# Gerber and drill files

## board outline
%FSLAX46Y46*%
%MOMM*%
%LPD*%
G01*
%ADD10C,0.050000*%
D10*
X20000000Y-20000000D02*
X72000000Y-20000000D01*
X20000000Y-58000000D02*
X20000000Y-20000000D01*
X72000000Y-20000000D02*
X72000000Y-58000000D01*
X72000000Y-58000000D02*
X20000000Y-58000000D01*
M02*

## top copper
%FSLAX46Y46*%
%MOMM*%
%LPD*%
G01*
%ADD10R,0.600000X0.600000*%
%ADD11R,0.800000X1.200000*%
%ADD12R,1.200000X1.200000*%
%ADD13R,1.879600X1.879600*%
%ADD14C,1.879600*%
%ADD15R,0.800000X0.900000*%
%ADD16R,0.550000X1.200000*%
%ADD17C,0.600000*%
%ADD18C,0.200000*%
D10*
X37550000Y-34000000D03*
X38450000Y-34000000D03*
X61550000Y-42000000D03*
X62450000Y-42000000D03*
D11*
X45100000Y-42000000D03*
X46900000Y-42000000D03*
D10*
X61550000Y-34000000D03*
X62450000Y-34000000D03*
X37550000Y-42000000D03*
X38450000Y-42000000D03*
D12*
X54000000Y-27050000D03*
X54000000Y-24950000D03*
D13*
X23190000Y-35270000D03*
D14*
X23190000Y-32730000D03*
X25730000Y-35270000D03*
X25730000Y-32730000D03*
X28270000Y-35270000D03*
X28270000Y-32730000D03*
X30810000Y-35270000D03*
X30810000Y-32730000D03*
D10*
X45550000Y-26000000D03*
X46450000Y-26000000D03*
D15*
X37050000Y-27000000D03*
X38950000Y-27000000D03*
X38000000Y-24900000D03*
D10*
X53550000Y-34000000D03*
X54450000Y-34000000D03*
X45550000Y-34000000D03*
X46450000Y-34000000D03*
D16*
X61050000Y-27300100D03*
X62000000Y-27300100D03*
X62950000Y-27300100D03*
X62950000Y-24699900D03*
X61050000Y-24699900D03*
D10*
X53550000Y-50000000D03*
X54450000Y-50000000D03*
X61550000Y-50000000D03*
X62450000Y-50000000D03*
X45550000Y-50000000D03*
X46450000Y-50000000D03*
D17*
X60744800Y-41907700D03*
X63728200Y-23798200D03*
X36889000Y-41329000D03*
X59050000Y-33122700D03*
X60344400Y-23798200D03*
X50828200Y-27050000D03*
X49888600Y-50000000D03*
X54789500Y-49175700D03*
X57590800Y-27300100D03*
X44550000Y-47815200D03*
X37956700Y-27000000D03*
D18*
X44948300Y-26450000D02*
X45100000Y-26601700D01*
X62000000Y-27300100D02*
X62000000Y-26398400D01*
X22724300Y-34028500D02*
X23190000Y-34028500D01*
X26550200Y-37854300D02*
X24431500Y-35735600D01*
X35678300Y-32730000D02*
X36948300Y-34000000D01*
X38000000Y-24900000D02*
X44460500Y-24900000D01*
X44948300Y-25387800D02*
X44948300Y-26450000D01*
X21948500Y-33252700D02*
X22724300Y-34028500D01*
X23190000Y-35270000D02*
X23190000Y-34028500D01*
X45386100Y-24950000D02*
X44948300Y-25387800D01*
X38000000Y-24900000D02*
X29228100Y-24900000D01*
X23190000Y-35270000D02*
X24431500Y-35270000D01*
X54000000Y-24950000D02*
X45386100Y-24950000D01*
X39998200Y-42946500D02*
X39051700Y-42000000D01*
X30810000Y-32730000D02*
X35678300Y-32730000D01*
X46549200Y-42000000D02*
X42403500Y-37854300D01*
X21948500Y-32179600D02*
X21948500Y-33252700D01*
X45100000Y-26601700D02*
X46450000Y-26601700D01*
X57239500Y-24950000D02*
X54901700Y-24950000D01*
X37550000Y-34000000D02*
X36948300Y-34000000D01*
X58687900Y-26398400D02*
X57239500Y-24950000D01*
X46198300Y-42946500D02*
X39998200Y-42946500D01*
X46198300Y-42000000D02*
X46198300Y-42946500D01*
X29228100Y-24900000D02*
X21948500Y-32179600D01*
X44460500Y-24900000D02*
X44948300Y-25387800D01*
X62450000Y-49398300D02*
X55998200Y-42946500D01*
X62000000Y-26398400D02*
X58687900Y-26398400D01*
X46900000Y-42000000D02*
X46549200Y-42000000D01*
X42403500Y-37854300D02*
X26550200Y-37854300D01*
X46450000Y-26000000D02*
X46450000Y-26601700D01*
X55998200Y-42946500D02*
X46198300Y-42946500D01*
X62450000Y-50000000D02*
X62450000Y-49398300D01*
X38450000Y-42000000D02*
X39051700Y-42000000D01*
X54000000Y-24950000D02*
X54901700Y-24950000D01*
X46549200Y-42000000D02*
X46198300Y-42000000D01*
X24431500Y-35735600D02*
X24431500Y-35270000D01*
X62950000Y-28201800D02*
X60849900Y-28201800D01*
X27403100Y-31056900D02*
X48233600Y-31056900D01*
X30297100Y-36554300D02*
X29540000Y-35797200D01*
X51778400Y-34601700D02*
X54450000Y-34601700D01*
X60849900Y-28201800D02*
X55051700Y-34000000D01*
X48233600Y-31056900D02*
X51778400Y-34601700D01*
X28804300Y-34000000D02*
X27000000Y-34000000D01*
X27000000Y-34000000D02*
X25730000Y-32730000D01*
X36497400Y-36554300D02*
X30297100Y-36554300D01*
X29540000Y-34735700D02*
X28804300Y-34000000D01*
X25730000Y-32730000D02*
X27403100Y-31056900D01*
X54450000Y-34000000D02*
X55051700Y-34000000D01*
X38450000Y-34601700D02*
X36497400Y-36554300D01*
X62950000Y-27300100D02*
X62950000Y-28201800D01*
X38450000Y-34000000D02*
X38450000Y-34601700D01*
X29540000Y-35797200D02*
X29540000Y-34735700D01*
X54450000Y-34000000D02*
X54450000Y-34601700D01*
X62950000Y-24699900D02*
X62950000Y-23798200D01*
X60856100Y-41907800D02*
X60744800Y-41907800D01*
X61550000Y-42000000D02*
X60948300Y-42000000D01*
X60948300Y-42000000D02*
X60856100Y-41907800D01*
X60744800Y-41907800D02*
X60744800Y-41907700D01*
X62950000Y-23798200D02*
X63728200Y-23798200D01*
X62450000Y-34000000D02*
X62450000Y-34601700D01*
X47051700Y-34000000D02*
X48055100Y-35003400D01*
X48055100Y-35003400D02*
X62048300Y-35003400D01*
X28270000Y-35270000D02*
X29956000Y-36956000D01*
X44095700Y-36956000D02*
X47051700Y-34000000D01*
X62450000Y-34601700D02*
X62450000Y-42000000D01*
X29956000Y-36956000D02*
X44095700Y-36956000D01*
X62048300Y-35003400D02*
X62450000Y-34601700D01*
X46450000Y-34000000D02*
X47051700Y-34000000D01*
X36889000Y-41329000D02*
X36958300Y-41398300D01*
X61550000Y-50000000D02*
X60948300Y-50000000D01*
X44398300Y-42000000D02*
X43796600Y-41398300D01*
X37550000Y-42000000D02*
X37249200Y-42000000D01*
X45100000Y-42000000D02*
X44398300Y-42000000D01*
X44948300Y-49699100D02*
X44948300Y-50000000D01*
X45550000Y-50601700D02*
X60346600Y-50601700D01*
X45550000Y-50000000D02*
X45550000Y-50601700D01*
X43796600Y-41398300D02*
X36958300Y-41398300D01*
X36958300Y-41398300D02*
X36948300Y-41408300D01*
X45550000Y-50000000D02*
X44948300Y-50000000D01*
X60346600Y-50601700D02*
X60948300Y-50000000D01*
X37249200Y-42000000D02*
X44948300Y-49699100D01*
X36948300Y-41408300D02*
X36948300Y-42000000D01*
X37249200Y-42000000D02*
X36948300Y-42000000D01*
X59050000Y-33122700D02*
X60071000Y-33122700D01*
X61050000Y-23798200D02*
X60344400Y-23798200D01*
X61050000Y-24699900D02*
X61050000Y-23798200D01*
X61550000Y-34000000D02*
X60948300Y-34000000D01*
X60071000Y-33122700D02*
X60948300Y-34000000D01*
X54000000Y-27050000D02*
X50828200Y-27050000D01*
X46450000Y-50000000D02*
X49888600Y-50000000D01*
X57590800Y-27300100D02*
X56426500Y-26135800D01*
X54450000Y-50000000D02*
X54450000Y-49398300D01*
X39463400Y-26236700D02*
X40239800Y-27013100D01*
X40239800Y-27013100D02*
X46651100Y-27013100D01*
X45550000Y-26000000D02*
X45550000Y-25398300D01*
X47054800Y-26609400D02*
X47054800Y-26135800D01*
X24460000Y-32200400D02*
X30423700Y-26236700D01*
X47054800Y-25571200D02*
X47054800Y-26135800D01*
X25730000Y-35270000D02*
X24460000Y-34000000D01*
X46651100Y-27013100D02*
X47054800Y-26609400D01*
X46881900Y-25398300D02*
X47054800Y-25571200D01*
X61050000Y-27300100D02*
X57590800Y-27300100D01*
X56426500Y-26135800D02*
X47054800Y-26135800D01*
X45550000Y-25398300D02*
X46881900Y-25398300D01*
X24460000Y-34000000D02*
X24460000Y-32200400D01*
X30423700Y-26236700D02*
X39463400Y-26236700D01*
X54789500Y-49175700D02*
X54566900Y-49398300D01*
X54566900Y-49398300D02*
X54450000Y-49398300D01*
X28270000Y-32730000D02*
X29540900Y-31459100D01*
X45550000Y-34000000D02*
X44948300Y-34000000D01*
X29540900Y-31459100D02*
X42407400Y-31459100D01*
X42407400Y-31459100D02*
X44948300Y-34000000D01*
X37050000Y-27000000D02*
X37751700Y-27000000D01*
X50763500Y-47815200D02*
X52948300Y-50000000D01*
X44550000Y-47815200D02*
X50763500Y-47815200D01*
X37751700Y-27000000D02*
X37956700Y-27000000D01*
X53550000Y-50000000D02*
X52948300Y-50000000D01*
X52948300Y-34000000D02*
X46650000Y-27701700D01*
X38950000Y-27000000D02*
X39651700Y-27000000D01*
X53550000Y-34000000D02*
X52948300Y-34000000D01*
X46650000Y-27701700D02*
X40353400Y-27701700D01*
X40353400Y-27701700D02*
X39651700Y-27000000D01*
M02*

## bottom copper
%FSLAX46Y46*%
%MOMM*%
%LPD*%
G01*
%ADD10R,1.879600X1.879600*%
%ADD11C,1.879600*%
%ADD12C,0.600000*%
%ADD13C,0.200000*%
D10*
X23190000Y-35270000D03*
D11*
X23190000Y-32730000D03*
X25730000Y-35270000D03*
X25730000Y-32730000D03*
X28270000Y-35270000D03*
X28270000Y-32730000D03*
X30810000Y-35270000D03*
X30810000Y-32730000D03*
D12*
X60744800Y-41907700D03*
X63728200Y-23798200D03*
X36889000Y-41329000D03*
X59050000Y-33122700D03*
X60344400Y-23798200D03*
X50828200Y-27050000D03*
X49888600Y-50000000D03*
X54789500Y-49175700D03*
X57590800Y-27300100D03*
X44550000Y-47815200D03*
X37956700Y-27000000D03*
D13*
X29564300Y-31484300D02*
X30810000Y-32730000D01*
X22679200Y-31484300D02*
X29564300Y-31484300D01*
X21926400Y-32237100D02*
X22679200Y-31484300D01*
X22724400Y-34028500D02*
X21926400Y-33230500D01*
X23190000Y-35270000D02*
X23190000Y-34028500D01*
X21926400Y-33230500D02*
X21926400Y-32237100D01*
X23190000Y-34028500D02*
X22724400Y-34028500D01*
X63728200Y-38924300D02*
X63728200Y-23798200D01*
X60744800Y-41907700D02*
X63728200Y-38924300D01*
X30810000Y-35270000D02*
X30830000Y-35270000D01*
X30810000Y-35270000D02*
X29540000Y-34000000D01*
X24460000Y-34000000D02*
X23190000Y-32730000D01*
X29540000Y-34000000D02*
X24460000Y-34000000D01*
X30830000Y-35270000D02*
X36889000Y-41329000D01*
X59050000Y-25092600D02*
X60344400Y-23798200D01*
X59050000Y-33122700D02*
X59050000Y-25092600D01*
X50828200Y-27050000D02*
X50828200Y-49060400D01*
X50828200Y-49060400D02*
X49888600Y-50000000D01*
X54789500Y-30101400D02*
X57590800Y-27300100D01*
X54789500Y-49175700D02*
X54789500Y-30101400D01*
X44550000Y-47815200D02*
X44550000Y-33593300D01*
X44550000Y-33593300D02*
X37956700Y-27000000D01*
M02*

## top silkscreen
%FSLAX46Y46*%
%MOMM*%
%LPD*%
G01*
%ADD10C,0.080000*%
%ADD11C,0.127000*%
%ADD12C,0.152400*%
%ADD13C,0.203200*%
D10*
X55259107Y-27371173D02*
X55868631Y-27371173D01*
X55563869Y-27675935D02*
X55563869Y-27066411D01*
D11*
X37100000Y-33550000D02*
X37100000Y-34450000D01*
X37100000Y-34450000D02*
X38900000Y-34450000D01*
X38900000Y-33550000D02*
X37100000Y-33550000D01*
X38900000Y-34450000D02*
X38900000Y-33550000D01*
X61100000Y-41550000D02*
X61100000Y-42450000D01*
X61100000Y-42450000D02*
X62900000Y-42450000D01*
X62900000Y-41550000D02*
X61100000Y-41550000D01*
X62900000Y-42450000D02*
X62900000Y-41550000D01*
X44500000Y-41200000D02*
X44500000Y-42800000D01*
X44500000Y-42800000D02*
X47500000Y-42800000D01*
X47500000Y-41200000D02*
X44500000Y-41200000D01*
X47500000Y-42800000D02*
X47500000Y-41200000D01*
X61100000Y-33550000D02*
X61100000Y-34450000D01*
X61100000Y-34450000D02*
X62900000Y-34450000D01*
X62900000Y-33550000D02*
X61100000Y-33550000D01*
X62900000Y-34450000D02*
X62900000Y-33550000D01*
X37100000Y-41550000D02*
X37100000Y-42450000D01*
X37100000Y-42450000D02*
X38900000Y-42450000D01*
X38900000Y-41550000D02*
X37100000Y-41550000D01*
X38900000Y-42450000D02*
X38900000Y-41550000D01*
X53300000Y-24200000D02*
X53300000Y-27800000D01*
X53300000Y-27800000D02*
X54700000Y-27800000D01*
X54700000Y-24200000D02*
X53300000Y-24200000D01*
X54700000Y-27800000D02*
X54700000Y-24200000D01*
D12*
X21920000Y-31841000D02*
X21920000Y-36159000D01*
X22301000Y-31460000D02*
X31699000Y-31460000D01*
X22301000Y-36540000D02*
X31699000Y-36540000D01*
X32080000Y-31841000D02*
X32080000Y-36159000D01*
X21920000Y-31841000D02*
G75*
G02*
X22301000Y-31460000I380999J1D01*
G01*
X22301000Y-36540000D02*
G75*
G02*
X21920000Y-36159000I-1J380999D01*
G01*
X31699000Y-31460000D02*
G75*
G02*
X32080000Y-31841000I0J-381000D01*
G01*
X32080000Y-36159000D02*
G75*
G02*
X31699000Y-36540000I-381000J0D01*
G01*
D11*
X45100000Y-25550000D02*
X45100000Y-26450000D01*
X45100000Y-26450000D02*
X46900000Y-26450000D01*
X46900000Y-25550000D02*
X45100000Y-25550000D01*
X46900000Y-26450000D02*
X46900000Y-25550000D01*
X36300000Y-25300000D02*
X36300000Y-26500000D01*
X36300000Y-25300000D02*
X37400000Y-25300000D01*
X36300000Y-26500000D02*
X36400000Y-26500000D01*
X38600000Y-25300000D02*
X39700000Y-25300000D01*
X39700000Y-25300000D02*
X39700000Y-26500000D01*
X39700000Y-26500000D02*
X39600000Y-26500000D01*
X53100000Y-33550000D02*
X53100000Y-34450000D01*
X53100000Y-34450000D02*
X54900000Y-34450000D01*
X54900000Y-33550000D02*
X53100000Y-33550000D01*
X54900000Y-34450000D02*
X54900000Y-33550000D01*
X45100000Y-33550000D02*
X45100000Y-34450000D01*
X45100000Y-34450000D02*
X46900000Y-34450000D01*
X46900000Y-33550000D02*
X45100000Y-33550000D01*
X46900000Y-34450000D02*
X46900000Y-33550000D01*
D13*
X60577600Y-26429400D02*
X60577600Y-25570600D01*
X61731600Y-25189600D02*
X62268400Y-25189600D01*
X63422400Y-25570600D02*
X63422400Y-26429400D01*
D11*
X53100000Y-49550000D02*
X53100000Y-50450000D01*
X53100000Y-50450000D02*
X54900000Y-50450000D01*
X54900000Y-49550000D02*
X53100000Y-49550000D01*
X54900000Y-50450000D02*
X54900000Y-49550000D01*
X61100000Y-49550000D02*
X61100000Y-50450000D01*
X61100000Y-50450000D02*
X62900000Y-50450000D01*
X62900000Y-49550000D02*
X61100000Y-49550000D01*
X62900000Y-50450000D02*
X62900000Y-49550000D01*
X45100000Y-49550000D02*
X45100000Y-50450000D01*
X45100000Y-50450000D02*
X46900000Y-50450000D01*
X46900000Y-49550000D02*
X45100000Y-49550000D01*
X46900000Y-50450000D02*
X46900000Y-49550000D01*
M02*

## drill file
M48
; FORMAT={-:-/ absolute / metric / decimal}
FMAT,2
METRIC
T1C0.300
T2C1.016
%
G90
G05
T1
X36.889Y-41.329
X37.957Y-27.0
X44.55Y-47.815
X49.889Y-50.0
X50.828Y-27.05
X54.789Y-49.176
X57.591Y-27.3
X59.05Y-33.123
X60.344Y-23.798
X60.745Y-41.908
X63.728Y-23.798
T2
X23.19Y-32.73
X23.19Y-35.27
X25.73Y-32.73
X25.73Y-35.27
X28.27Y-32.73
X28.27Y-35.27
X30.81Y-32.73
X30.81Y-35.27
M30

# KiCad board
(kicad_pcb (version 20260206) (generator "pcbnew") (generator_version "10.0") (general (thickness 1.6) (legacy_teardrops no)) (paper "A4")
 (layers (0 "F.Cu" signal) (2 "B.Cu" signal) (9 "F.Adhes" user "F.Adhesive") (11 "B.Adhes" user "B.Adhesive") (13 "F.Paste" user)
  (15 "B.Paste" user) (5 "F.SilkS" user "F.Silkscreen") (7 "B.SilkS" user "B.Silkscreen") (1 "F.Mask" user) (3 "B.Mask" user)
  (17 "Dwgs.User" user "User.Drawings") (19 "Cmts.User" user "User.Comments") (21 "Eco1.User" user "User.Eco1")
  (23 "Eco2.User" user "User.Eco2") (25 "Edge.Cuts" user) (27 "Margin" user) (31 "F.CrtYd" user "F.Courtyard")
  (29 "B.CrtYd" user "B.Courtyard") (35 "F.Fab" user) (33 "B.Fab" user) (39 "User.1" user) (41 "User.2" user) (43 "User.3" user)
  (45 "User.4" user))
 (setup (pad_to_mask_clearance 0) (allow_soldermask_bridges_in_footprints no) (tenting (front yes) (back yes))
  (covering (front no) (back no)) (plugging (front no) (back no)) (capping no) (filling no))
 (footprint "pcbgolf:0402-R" (layer "F.Cu") (at 38 34)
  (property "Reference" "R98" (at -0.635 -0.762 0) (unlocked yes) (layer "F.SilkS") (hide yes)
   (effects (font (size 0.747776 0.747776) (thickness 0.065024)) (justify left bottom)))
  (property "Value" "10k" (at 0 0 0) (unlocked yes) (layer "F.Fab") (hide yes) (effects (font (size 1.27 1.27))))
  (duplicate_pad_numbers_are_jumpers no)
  (fp_line (start -0.9 -0.45) (end -0.9 0.45) (stroke (width 0.127) (type solid)) (layer "F.SilkS"))
  (fp_line (start -0.9 0.45) (end 0.9 0.45) (stroke (width 0.127) (type solid)) (layer "F.SilkS"))
  (fp_line (start 0.9 -0.45) (end -0.9 -0.45) (stroke (width 0.127) (type solid)) (layer "F.SilkS"))
  (fp_line (start 0.9 0.45) (end 0.9 -0.45) (stroke (width 0.127) (type solid)) (layer "F.SilkS"))
  (pad "1" smd rect (at -0.45 0) (size 0.6 0.6) (layers "F.Cu" "F.Mask" "F.Paste") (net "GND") (solder_mask_margin 0.0508)
   (solder_paste_margin 0) (thermal_bridge_angle 0))
  (pad "2" smd rect (at 0.45 0) (size 0.6 0.6) (layers "F.Cu" "F.Mask" "F.Paste") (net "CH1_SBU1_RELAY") (solder_mask_margin 0.0508)
   (solder_paste_margin 0) (thermal_bridge_angle 0)))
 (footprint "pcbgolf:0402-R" (layer "F.Cu") (at 62 42)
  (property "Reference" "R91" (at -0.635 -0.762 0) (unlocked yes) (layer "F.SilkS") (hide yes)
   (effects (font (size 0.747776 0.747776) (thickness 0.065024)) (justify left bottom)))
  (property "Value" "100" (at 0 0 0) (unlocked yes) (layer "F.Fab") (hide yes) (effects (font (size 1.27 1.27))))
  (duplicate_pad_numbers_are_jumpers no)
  (fp_line (start -0.9 -0.45) (end -0.9 0.45) (stroke (width 0.127) (type solid)) (layer "F.SilkS"))
  (fp_line (start -0.9 0.45) (end 0.9 0.45) (stroke (width 0.127) (type solid)) (layer "F.SilkS"))
  (fp_line (start 0.9 -0.45) (end -0.9 -0.45) (stroke (width 0.127) (type solid)) (layer "F.SilkS"))
  (fp_line (start 0.9 0.45) (end 0.9 -0.45) (stroke (width 0.127) (type solid)) (layer "F.SilkS"))
  (pad "1" smd rect (at -0.45 0) (size 0.6 0.6) (layers "F.Cu" "F.Mask" "F.Paste") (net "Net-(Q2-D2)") (solder_mask_margin 0.0508)
   (solder_paste_margin 0) (thermal_bridge_angle 0))
  (pad "2" smd rect (at 0.45 0) (size 0.6 0.6) (layers "F.Cu" "F.Mask" "F.Paste") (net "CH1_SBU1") (solder_mask_margin 0.0508)
   (solder_paste_margin 0) (thermal_bridge_angle 0)))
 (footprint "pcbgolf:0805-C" (layer "F.Cu") (at 46 42)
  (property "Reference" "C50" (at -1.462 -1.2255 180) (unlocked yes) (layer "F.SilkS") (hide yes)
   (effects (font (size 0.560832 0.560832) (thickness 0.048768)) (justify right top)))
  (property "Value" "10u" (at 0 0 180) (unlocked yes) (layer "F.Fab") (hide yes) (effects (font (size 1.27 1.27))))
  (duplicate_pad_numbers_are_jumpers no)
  (fp_line (start -1.5 -0.8) (end -1.5 0.8) (stroke (width 0.127) (type solid)) (layer "F.SilkS"))
  (fp_line (start -1.5 0.8) (end 1.5 0.8) (stroke (width 0.127) (type solid)) (layer "F.SilkS"))
  (fp_line (start 1.5 -0.8) (end -1.5 -0.8) (stroke (width 0.127) (type solid)) (layer "F.SilkS"))
  (fp_line (start 1.5 0.8) (end 1.5 -0.8) (stroke (width 0.127) (type solid)) (layer "F.SilkS"))
  (pad "1" smd rect (at -0.9 0) (size 0.8 1.2) (layers "F.Cu" "F.Mask" "F.Paste") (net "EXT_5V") (solder_mask_margin 0.0508)
   (solder_paste_margin 0) (thermal_bridge_angle 0))
  (pad "2" smd rect (at 0.9 0) (size 0.8 1.2) (layers "F.Cu" "F.Mask" "F.Paste") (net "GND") (solder_mask_margin 0.0508)
   (solder_paste_margin 0) (thermal_bridge_angle 0)))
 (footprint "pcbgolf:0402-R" (layer "F.Cu") (at 62 34)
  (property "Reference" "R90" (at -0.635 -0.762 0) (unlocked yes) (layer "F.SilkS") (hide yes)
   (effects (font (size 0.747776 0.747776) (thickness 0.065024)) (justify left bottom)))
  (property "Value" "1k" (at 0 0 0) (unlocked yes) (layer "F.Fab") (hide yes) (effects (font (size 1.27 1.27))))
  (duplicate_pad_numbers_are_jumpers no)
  (fp_line (start -0.9 -0.45) (end -0.9 0.45) (stroke (width 0.127) (type solid)) (layer "F.SilkS"))
  (fp_line (start -0.9 0.45) (end 0.9 0.45) (stroke (width 0.127) (type solid)) (layer "F.SilkS"))
  (fp_line (start 0.9 -0.45) (end -0.9 -0.45) (stroke (width 0.127) (type solid)) (layer "F.SilkS"))
  (fp_line (start 0.9 0.45) (end 0.9 -0.45) (stroke (width 0.127) (type solid)) (layer "F.SilkS"))
  (pad "1" smd rect (at -0.45 0) (size 0.6 0.6) (layers "F.Cu" "F.Mask" "F.Paste") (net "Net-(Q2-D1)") (solder_mask_margin 0.0508)
   (solder_paste_margin 0) (thermal_bridge_angle 0))
  (pad "2" smd rect (at 0.45 0) (size 0.6 0.6) (layers "F.Cu" "F.Mask" "F.Paste") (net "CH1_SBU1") (solder_mask_margin 0.0508)
   (solder_paste_margin 0) (thermal_bridge_angle 0)))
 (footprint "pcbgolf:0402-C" (layer "F.Cu") (at 38 42)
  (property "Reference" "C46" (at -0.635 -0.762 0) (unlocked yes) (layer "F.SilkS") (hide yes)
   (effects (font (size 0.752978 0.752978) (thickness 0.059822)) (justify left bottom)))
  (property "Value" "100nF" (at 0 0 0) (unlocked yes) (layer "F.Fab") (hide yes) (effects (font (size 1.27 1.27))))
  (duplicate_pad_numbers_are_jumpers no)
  (fp_line (start -0.9 -0.45) (end -0.9 0.45) (stroke (width 0.127) (type solid)) (layer "F.SilkS"))
  (fp_line (start -0.9 0.45) (end 0.9 0.45) (stroke (width 0.127) (type solid)) (layer "F.SilkS"))
  (fp_line (start 0.9 -0.45) (end -0.9 -0.45) (stroke (width 0.127) (type solid)) (layer "F.SilkS"))
  (fp_line (start 0.9 0.45) (end 0.9 -0.45) (stroke (width 0.127) (type solid)) (layer "F.SilkS"))
  (pad "1" smd rect (at -0.45 0) (size 0.6 0.6) (layers "F.Cu" "F.Mask" "F.Paste") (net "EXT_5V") (solder_mask_margin 0.0508)
   (solder_paste_margin 0) (thermal_bridge_angle 0))
  (pad "2" smd rect (at 0.45 0) (size 0.6 0.6) (layers "F.Cu" "F.Mask" "F.Paste") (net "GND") (solder_mask_margin 0.0508)
   (solder_paste_margin 0) (thermal_bridge_angle 0)))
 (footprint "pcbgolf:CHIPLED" (layer "F.Cu") (at 54 26)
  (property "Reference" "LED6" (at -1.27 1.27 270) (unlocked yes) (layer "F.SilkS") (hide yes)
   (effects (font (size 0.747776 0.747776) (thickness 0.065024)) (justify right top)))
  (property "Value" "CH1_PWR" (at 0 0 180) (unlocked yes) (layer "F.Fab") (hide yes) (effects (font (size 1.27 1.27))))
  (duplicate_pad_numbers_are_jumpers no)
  (fp_line (start -0.7 -1.8) (end -0.7 1.8) (stroke (width 0.127) (type solid)) (layer "F.SilkS"))
  (fp_line (start -0.7 1.8) (end 0.7 1.8) (stroke (width 0.127) (type solid)) (layer "F.SilkS"))
  (fp_line (start 0.7 -1.8) (end -0.7 -1.8) (stroke (width 0.127) (type solid)) (layer "F.SilkS"))
  (fp_line (start 0.7 1.8) (end 0.7 -1.8) (stroke (width 0.127) (type solid)) (layer "F.SilkS"))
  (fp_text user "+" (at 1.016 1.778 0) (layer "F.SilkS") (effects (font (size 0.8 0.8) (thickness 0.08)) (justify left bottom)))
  (pad "A" smd rect (at 0 1.05) (size 1.2 1.2) (layers "F.Cu" "F.Mask" "F.Paste") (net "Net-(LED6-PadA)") (solder_mask_margin 0.0508)
   (solder_paste_margin 0) (thermal_bridge_angle 0))
  (pad "C" smd rect (at 0 -1.05) (size 1.2 1.2) (layers "F.Cu" "F.Mask" "F.Paste") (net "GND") (solder_mask_margin 0.0508)
   (solder_paste_margin 0) (thermal_bridge_angle 0)))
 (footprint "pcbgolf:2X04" (layer "F.Cu") (at 27 34)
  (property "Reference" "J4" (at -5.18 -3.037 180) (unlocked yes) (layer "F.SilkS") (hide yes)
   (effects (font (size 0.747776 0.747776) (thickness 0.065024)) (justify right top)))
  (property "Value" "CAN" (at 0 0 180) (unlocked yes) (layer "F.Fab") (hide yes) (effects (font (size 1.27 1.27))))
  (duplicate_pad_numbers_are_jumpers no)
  (fp_line (start -5.08 -2.159) (end -5.08 2.159) (stroke (width 0.1524) (type solid)) (layer "F.SilkS"))
  (fp_line (start -4.699 -2.54) (end 4.699 -2.54) (stroke (width 0.1524) (type solid)) (layer "F.SilkS"))
  (fp_line (start -4.699 2.54) (end 4.699 2.54) (stroke (width 0.1524) (type solid)) (layer "F.SilkS"))
  (fp_line (start 5.08 -2.159) (end 5.08 2.159) (stroke (width 0.1524) (type solid)) (layer "F.SilkS"))
  (fp_arc (start -5.08 -2.159) (mid -4.968408 -2.428408) (end -4.699 -2.54) (stroke (width 0.1524) (type solid)) (layer "F.SilkS"))
  (fp_arc (start -4.699 2.54) (mid -4.968408 2.428408) (end -5.08 2.159) (stroke (width 0.1524) (type solid)) (layer "F.SilkS"))
  (fp_arc (start 4.699 -2.54) (mid 4.968408 -2.428408) (end 5.08 -2.159) (stroke (width 0.1524) (type solid)) (layer "F.SilkS"))
  (fp_arc (start 5.08 2.159) (mid 4.968408 2.428408) (end 4.699 2.54) (stroke (width 0.1524) (type solid)) (layer "F.SilkS"))
  (pad "1" thru_hole rect (at -3.81 1.27 90) (size 1.8796 1.8796) (drill 1.016) (layers "*.Cu" "*.Mask") (remove_unused_layers no)
   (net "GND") (solder_mask_margin 0.0508) (thermal_bridge_angle 0))
  (pad "2" thru_hole circle (at -3.81 -1.27 90) (size 1.8796 1.8796) (drill 1.016) (layers "*.Cu" "*.Mask") (remove_unused_layers no)
   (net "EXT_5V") (solder_mask_margin 0.0508) (thermal_bridge_angle 0))
  (pad "3" thru_hole circle (at -1.27 1.27 90) (size 1.8796 1.8796) (drill 1.016) (layers "*.Cu" "*.Mask") (remove_unused_layers no)
   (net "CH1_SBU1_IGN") (solder_mask_margin 0.0508) (thermal_bridge_angle 0))
  (pad "4" thru_hole circle (at -1.27 -1.27 90) (size 1.8796 1.8796) (drill 1.016) (layers "*.Cu" "*.Mask") (remove_unused_layers no)
   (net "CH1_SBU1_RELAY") (solder_mask_margin 0.0508) (thermal_bridge_angle 0))
  (pad "5" thru_hole circle (at 1.27 1.27 90) (size 1.8796 1.8796) (drill 1.016) (layers "*.Cu" "*.Mask") (remove_unused_layers no)
   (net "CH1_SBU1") (solder_mask_margin 0.0508) (thermal_bridge_angle 0))
  (pad "6" thru_hole circle (at 1.27 -1.27 90) (size 1.8796 1.8796) (drill 1.016) (layers "*.Cu" "*.Mask") (remove_unused_layers no)
   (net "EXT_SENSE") (solder_mask_margin 0.0508) (thermal_bridge_angle 0))
  (pad "7" thru_hole circle (at 3.81 1.27 90) (size 1.8796 1.8796) (drill 1.016) (layers "*.Cu" "*.Mask") (remove_unused_layers no)
   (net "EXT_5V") (solder_mask_margin 0.0508) (thermal_bridge_angle 0))
  (pad "8" thru_hole circle (at 3.81 -1.27 90) (size 1.8796 1.8796) (drill 1.016) (layers "*.Cu" "*.Mask") (remove_unused_layers no)
   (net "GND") (solder_mask_margin 0.0508) (thermal_bridge_angle 0)))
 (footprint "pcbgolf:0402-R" (layer "F.Cu") (at 46 26)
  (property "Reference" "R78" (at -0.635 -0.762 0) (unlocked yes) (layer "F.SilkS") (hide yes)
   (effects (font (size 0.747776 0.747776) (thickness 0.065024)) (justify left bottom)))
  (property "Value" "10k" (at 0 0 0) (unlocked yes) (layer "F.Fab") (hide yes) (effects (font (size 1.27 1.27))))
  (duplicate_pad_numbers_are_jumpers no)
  (fp_line (start -0.9 -0.45) (end -0.9 0.45) (stroke (width 0.127) (type solid)) (layer "F.SilkS"))
  (fp_line (start -0.9 0.45) (end 0.9 0.45) (stroke (width 0.127) (type solid)) (layer "F.SilkS"))
  (fp_line (start 0.9 -0.45) (end -0.9 -0.45) (stroke (width 0.127) (type solid)) (layer "F.SilkS"))
  (fp_line (start 0.9 0.45) (end 0.9 -0.45) (stroke (width 0.127) (type solid)) (layer "F.SilkS"))
  (pad "1" smd rect (at -0.45 0) (size 0.6 0.6) (layers "F.Cu" "F.Mask" "F.Paste") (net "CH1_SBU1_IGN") (solder_mask_margin 0.0508)
   (solder_paste_margin 0) (thermal_bridge_angle 0))
  (pad "2" smd rect (at 0.45 0) (size 0.6 0.6) (layers "F.Cu" "F.Mask" "F.Paste") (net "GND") (solder_mask_margin 0.0508)
   (solder_paste_margin 0) (thermal_bridge_angle 0)))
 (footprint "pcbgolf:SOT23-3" (layer "F.Cu") (at 38 26)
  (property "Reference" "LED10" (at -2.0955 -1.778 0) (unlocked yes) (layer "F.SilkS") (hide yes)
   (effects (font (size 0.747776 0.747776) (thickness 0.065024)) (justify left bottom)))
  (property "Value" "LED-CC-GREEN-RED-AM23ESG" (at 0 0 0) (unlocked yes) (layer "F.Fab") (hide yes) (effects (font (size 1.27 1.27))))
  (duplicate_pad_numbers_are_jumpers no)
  (fp_line (start -1.7 -0.7) (end -1.7 0.5) (stroke (width 0.127) (type solid)) (layer "F.SilkS"))
  (fp_line (start -1.7 -0.7) (end -0.6 -0.7) (stroke (width 0.127) (type solid)) (layer "F.SilkS"))
  (fp_line (start -1.7 0.5) (end -1.6 0.5) (stroke (width 0.127) (type solid)) (layer "F.SilkS"))
  (fp_line (start 0.6 -0.7) (end 1.7 -0.7) (stroke (width 0.127) (type solid)) (layer "F.SilkS"))
  (fp_line (start 1.7 -0.7) (end 1.7 0.5) (stroke (width 0.127) (type solid)) (layer "F.SilkS"))
  (fp_line (start 1.7 0.5) (end 1.6 0.5) (stroke (width 0.127) (type solid)) (layer "F.SilkS"))
  (pad "1" smd rect (at -0.95 1) (size 0.8 0.9) (layers "F.Cu" "F.Mask" "F.Paste") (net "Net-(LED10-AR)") (solder_mask_margin 0.0508)
   (solder_paste_margin 0) (thermal_bridge_angle 0))
  (pad "2" smd rect (at 0.95 1) (size 0.8 0.9) (layers "F.Cu" "F.Mask" "F.Paste") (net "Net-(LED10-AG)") (solder_mask_margin 0.0508)
   (solder_paste_margin 0) (thermal_bridge_angle 0))
  (pad "3" smd rect (at 0 -1.1) (size 0.8 0.9) (layers "F.Cu" "F.Mask" "F.Paste") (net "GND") (solder_mask_margin 0.0508)
   (solder_paste_margin 0) (thermal_bridge_angle 0)))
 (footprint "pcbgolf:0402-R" (layer "F.Cu") (at 54 34)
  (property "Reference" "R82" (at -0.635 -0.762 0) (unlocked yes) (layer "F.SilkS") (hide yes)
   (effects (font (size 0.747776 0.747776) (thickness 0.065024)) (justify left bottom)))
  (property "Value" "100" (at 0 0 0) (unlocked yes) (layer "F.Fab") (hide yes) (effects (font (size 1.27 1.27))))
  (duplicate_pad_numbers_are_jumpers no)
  (fp_line (start -0.9 -0.45) (end -0.9 0.45) (stroke (width 0.127) (type solid)) (layer "F.SilkS"))
  (fp_line (start -0.9 0.45) (end 0.9 0.45) (stroke (width 0.127) (type solid)) (layer "F.SilkS"))
  (fp_line (start 0.9 -0.45) (end -0.9 -0.45) (stroke (width 0.127) (type solid)) (layer "F.SilkS"))
  (fp_line (start 0.9 0.45) (end 0.9 -0.45) (stroke (width 0.127) (type solid)) (layer "F.SilkS"))
  (pad "1" smd rect (at -0.45 0) (size 0.6 0.6) (layers "F.Cu" "F.Mask" "F.Paste") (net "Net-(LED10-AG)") (solder_mask_margin 0.0508)
   (solder_paste_margin 0) (thermal_bridge_angle 0))
  (pad "2" smd rect (at 0.45 0) (size 0.6 0.6) (layers "F.Cu" "F.Mask" "F.Paste") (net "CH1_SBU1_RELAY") (solder_mask_margin 0.0508)
   (solder_paste_margin 0) (thermal_bridge_angle 0)))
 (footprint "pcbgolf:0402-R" (layer "F.Cu") (at 46 34)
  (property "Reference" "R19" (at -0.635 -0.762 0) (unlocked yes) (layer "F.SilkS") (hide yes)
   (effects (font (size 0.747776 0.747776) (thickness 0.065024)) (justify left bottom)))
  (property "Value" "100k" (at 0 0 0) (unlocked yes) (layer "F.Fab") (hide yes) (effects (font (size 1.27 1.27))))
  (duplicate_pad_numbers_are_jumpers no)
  (fp_line (start -0.9 -0.45) (end -0.9 0.45) (stroke (width 0.127) (type solid)) (layer "F.SilkS"))
  (fp_line (start -0.9 0.45) (end 0.9 0.45) (stroke (width 0.127) (type solid)) (layer "F.SilkS"))
  (fp_line (start 0.9 -0.45) (end -0.9 -0.45) (stroke (width 0.127) (type solid)) (layer "F.SilkS"))
  (fp_line (start 0.9 0.45) (end 0.9 -0.45) (stroke (width 0.127) (type solid)) (layer "F.SilkS"))
  (pad "1" smd rect (at -0.45 0) (size 0.6 0.6) (layers "F.Cu" "F.Mask" "F.Paste") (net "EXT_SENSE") (solder_mask_margin 0.0508)
   (solder_paste_margin 0) (thermal_bridge_angle 0))
  (pad "2" smd rect (at 0.45 0) (size 0.6 0.6) (layers "F.Cu" "F.Mask" "F.Paste") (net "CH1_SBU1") (solder_mask_margin 0.0508)
   (solder_paste_margin 0) (thermal_bridge_angle 0)))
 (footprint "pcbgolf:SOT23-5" (layer "F.Cu") (at 62 26)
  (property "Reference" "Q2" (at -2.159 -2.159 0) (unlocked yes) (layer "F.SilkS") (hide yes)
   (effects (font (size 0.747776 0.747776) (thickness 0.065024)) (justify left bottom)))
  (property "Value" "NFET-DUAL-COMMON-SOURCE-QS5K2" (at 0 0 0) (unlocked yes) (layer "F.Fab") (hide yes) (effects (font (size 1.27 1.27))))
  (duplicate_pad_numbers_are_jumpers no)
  (fp_line (start -1.4224 0.4294) (end -1.4224 -0.4294) (stroke (width 0.2032) (type solid)) (layer "F.SilkS"))
  (fp_line (start -0.2684 -0.8104) (end 0.2684 -0.8104) (stroke (width 0.2032) (type solid)) (layer "F.SilkS"))
  (fp_line (start 1.4224 -0.4294) (end 1.4224 0.4294) (stroke (width 0.2032) (type solid)) (layer "F.SilkS"))
  (pad "1" smd rect (at -0.95 1.3001) (size 0.55 1.2) (layers "F.Cu" "F.Mask" "F.Paste") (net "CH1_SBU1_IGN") (solder_mask_margin 0.0508)
   (solder_paste_margin 0) (thermal_bridge_angle 0))
  (pad "2" smd rect (at 0 1.3001) (size 0.55 1.2) (layers "F.Cu" "F.Mask" "F.Paste") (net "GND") (solder_mask_margin 0.0508)
   (solder_paste_margin 0) (thermal_bridge_angle 0))
  (pad "3" smd rect (at 0.95 1.3001) (size 0.55 1.2) (layers "F.Cu" "F.Mask" "F.Paste") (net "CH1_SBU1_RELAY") (solder_mask_margin 0.0508)
   (solder_paste_margin 0) (thermal_bridge_angle 0))
  (pad "4" smd rect (at 0.95 -1.3001) (size 0.55 1.2) (layers "F.Cu" "F.Mask" "F.Paste") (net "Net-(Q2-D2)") (solder_mask_margin 0.0508)
   (solder_paste_margin 0) (thermal_bridge_angle 0))
  (pad "5" smd rect (at -0.95 -1.3001) (size 0.55 1.2) (layers "F.Cu" "F.Mask" "F.Paste") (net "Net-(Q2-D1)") (solder_mask_margin 0.0508)
   (solder_paste_margin 0) (thermal_bridge_angle 0)))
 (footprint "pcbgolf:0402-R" (layer "F.Cu") (at 54 50)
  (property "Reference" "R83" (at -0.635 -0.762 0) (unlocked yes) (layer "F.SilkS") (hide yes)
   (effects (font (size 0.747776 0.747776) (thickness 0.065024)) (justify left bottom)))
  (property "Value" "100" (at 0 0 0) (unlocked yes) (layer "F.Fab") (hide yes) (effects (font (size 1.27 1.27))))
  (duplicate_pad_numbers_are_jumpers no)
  (fp_line (start -0.9 -0.45) (end -0.9 0.45) (stroke (width 0.127) (type solid)) (layer "F.SilkS"))
  (fp_line (start -0.9 0.45) (end 0.9 0.45) (stroke (width 0.127) (type solid)) (layer "F.SilkS"))
  (fp_line (start 0.9 -0.45) (end -0.9 -0.45) (stroke (width 0.127) (type solid)) (layer "F.SilkS"))
  (fp_line (start 0.9 0.45) (end 0.9 -0.45) (stroke (width 0.127) (type solid)) (layer "F.SilkS"))
  (pad "1" smd rect (at -0.45 0) (size 0.6 0.6) (layers "F.Cu" "F.Mask" "F.Paste") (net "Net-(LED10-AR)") (solder_mask_margin 0.0508)
   (solder_paste_margin 0) (thermal_bridge_angle 0))
  (pad "2" smd rect (at 0.45 0) (size 0.6 0.6) (layers "F.Cu" "F.Mask" "F.Paste") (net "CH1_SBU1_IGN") (solder_mask_margin 0.0508)
   (solder_paste_margin 0) (thermal_bridge_angle 0)))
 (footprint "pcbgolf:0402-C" (layer "F.Cu") (at 62 50)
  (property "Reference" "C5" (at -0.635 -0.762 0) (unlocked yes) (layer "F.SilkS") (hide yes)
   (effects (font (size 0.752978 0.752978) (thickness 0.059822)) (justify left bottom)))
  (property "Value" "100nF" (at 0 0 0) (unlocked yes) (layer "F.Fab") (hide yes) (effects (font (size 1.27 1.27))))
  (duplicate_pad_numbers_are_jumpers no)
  (fp_line (start -0.9 -0.45) (end -0.9 0.45) (stroke (width 0.127) (type solid)) (layer "F.SilkS"))
  (fp_line (start -0.9 0.45) (end 0.9 0.45) (stroke (width 0.127) (type solid)) (layer "F.SilkS"))
  (fp_line (start 0.9 -0.45) (end -0.9 -0.45) (stroke (width 0.127) (type solid)) (layer "F.SilkS"))
  (fp_line (start 0.9 0.45) (end 0.9 -0.45) (stroke (width 0.127) (type solid)) (layer "F.SilkS"))
  (pad "1" smd rect (at -0.45 0) (size 0.6 0.6) (layers "F.Cu" "F.Mask" "F.Paste") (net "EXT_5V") (solder_mask_margin 0.0508)
   (solder_paste_margin 0) (thermal_bridge_angle 0))
  (pad "2" smd rect (at 0.45 0) (size 0.6 0.6) (layers "F.Cu" "F.Mask" "F.Paste") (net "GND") (solder_mask_margin 0.0508)
   (solder_paste_margin 0) (thermal_bridge_angle 0)))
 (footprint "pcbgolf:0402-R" (layer "F.Cu") (at 46 50)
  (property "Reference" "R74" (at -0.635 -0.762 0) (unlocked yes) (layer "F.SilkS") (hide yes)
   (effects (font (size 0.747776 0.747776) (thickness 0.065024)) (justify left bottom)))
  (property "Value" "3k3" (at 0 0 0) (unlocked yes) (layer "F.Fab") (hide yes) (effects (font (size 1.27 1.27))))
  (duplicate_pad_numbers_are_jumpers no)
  (fp_line (start -0.9 -0.45) (end -0.9 0.45) (stroke (width 0.127) (type solid)) (layer "F.SilkS"))
  (fp_line (start -0.9 0.45) (end 0.9 0.45) (stroke (width 0.127) (type solid)) (layer "F.SilkS"))
  (fp_line (start 0.9 -0.45) (end -0.9 -0.45) (stroke (width 0.127) (type solid)) (layer "F.SilkS"))
  (fp_line (start 0.9 0.45) (end 0.9 -0.45) (stroke (width 0.127) (type solid)) (layer "F.SilkS"))
  (pad "1" smd rect (at -0.45 0) (size 0.6 0.6) (layers "F.Cu" "F.Mask" "F.Paste") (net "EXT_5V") (solder_mask_margin 0.0508)
   (solder_paste_margin 0) (thermal_bridge_angle 0))
  (pad "2" smd rect (at 0.45 0) (size 0.6 0.6) (layers "F.Cu" "F.Mask" "F.Paste") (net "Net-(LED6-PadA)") (solder_mask_margin 0.0508)
   (solder_paste_margin 0) (thermal_bridge_angle 0)))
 (gr_line (start 20 20) (end 72 20) (stroke (width 0.05) (type default)) (layer "Edge.Cuts"))
 (gr_line (start 20 58) (end 20 20) (stroke (width 0.05) (type default)) (layer "Edge.Cuts"))
 (gr_line (start 72 20) (end 72 58) (stroke (width 0.05) (type default)) (layer "Edge.Cuts"))
 (gr_line (start 72 58) (end 20 58) (stroke (width 0.05) (type default)) (layer "Edge.Cuts"))
 (segment (start 44.9483 26.45) (end 45.1 26.6017) (width 0.2) (layer "F.Cu") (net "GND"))
 (segment (start 62 27.3001) (end 62 26.3984) (width 0.2) (layer "F.Cu") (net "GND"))
 (segment (start 22.7243 34.0285) (end 23.19 34.0285) (width 0.2) (layer "F.Cu") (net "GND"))
 (segment (start 26.5502 37.8543) (end 24.4315 35.7356) (width 0.2) (layer "F.Cu") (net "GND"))
 (segment (start 35.6783 32.73) (end 36.9483 34) (width 0.2) (layer "F.Cu") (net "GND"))
 (segment (start 38 24.9) (end 44.4605 24.9) (width 0.2) (layer "F.Cu") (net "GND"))
 (segment (start 44.9483 25.3878) (end 44.9483 26.45) (width 0.2) (layer "F.Cu") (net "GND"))
 (segment (start 21.9485 33.2527) (end 22.7243 34.0285) (width 0.2) (layer "F.Cu") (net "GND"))
 (segment (start 23.19 35.27) (end 23.19 34.0285) (width 0.2) (layer "F.Cu") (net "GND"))
 (segment (start 45.3861 24.95) (end 44.9483 25.3878) (width 0.2) (layer "F.Cu") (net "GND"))
 (segment (start 38 24.9) (end 29.2281 24.9) (width 0.2) (layer "F.Cu") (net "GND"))
 (segment (start 23.19 35.27) (end 24.4315 35.27) (width 0.2) (layer "F.Cu") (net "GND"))
 (segment (start 54 24.95) (end 45.3861 24.95) (width 0.2) (layer "F.Cu") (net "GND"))
 (segment (start 39.9982 42.9465) (end 39.0517 42) (width 0.2) (layer "F.Cu") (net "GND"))
 (segment (start 30.81 32.73) (end 35.6783 32.73) (width 0.2) (layer "F.Cu") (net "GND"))
 (segment (start 46.5492 42) (end 42.4035 37.8543) (width 0.2) (layer "F.Cu") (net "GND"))
 (segment (start 21.9485 32.1796) (end 21.9485 33.2527) (width 0.2) (layer "F.Cu") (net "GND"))
 (segment (start 45.1 26.6017) (end 46.45 26.6017) (width 0.2) (layer "F.Cu") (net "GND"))
 (segment (start 57.2395 24.95) (end 54.9017 24.95) (width 0.2) (layer "F.Cu") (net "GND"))
 (segment (start 37.55 34) (end 36.9483 34) (width 0.2) (layer "F.Cu") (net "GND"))
 (segment (start 58.6879 26.3984) (end 57.2395 24.95) (width 0.2) (layer "F.Cu") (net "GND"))
 (segment (start 46.1983 42.9465) (end 39.9982 42.9465) (width 0.2) (layer "F.Cu") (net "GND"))
 (segment (start 46.1983 42) (end 46.1983 42.9465) (width 0.2) (layer "F.Cu") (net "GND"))
 (segment (start 29.2281 24.9) (end 21.9485 32.1796) (width 0.2) (layer "F.Cu") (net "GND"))
 (segment (start 44.4605 24.9) (end 44.9483 25.3878) (width 0.2) (layer "F.Cu") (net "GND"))
 (segment (start 62.45 49.3983) (end 55.9982 42.9465) (width 0.2) (layer "F.Cu") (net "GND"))
 (segment (start 62 26.3984) (end 58.6879 26.3984) (width 0.2) (layer "F.Cu") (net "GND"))
 (segment (start 46.9 42) (end 46.5492 42) (width 0.2) (layer "F.Cu") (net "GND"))
 (segment (start 42.4035 37.8543) (end 26.5502 37.8543) (width 0.2) (layer "F.Cu") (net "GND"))
 (segment (start 46.45 26) (end 46.45 26.6017) (width 0.2) (layer "F.Cu") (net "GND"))
 (segment (start 55.9982 42.9465) (end 46.1983 42.9465) (width 0.2) (layer "F.Cu") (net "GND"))
 (segment (start 62.45 50) (end 62.45 49.3983) (width 0.2) (layer "F.Cu") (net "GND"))
 (segment (start 38.45 42) (end 39.0517 42) (width 0.2) (layer "F.Cu") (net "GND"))
 (segment (start 54 24.95) (end 54.9017 24.95) (width 0.2) (layer "F.Cu") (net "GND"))
 (segment (start 46.5492 42) (end 46.1983 42) (width 0.2) (layer "F.Cu") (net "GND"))
 (segment (start 24.4315 35.7356) (end 24.4315 35.27) (width 0.2) (layer "F.Cu") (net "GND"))
 (segment (start 29.5643 31.4843) (end 30.81 32.73) (width 0.2) (layer "B.Cu") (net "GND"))
 (segment (start 22.6792 31.4843) (end 29.5643 31.4843) (width 0.2) (layer "B.Cu") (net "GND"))
 (segment (start 21.9264 32.2371) (end 22.6792 31.4843) (width 0.2) (layer "B.Cu") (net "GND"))
 (segment (start 22.7244 34.0285) (end 21.9264 33.2305) (width 0.2) (layer "B.Cu") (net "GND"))
 (segment (start 23.19 35.27) (end 23.19 34.0285) (width 0.2) (layer "B.Cu") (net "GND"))
 (segment (start 21.9264 33.2305) (end 21.9264 32.2371) (width 0.2) (layer "B.Cu") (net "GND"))
 (segment (start 23.19 34.0285) (end 22.7244 34.0285) (width 0.2) (layer "B.Cu") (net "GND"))
 (segment (start 62.95 28.2018) (end 60.8499 28.2018) (width 0.2) (layer "F.Cu") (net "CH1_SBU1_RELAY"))
 (segment (start 27.4031 31.0569) (end 48.2336 31.0569) (width 0.2) (layer "F.Cu") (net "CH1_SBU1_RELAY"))
 (segment (start 30.2971 36.5543) (end 29.54 35.7972) (width 0.2) (layer "F.Cu") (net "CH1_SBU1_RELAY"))
 (segment (start 51.7784 34.6017) (end 54.45 34.6017) (width 0.2) (layer "F.Cu") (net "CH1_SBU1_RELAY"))
 (segment (start 60.8499 28.2018) (end 55.0517 34) (width 0.2) (layer "F.Cu") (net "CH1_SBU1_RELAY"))
 (segment (start 48.2336 31.0569) (end 51.7784 34.6017) (width 0.2) (layer "F.Cu") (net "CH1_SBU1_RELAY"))
 (segment (start 28.8043 34) (end 27 34) (width 0.2) (layer "F.Cu") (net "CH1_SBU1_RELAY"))
 (segment (start 27 34) (end 25.73 32.73) (width 0.2) (layer "F.Cu") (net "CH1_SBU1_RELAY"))
 (segment (start 36.4974 36.5543) (end 30.2971 36.5543) (width 0.2) (layer "F.Cu") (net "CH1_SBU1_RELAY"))
 (segment (start 29.54 34.7357) (end 28.8043 34) (width 0.2) (layer "F.Cu") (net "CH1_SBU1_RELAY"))
 (segment (start 25.73 32.73) (end 27.4031 31.0569) (width 0.2) (layer "F.Cu") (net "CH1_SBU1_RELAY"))
 (segment (start 54.45 34) (end 55.0517 34) (width 0.2) (layer "F.Cu") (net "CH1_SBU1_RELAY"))
 (segment (start 38.45 34.6017) (end 36.4974 36.5543) (width 0.2) (layer "F.Cu") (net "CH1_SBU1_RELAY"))
 (segment (start 62.95 27.3001) (end 62.95 28.2018) (width 0.2) (layer "F.Cu") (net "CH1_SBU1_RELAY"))
 (segment (start 38.45 34) (end 38.45 34.6017) (width 0.2) (layer "F.Cu") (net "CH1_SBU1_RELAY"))
 (segment (start 29.54 35.7972) (end 29.54 34.7357) (width 0.2) (layer "F.Cu") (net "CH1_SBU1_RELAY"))
 (segment (start 54.45 34) (end 54.45 34.6017) (width 0.2) (layer "F.Cu") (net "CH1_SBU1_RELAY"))
 (segment (start 62.95 24.6999) (end 62.95 23.7982) (width 0.2) (layer "F.Cu") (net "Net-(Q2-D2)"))
 (segment (start 60.8561 41.9078) (end 60.7448 41.9078) (width 0.2) (layer "F.Cu") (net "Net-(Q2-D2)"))
 (segment (start 61.55 42) (end 60.9483 42) (width 0.2) (layer "F.Cu") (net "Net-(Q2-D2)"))
 (segment (start 60.9483 42) (end 60.8561 41.9078) (width 0.2) (layer "F.Cu") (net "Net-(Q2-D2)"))
 (segment (start 60.7448 41.9078) (end 60.7448 41.9077) (width 0.2) (layer "F.Cu") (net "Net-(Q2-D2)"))
 (segment (start 62.95 23.7982) (end 63.7282 23.7982) (width 0.2) (layer "F.Cu") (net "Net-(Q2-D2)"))
 (via (at 60.7448 41.9077) (size 0.6) (drill 0.3) (layers "F.Cu" "B.Cu") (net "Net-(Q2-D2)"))
 (via (at 63.7282 23.7982) (size 0.6) (drill 0.3) (layers "F.Cu" "B.Cu") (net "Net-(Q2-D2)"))
 (segment (start 63.7282 38.9243) (end 63.7282 23.7982) (width 0.2) (layer "B.Cu") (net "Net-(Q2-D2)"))
 (segment (start 60.7448 41.9077) (end 63.7282 38.9243) (width 0.2) (layer "B.Cu") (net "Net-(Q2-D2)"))
 (segment (start 62.45 34) (end 62.45 34.6017) (width 0.2) (layer "F.Cu") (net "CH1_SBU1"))
 (segment (start 47.0517 34) (end 48.0551 35.0034) (width 0.2) (layer "F.Cu") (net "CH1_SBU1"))
 (segment (start 48.0551 35.0034) (end 62.0483 35.0034) (width 0.2) (layer "F.Cu") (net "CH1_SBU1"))
 (segment (start 28.27 35.27) (end 29.956 36.956) (width 0.2) (layer "F.Cu") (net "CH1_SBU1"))
 (segment (start 44.0957 36.956) (end 47.0517 34) (width 0.2) (layer "F.Cu") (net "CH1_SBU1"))
 (segment (start 62.45 34.6017) (end 62.45 42) (width 0.2) (layer "F.Cu") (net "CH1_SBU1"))
 (segment (start 29.956 36.956) (end 44.0957 36.956) (width 0.2) (layer "F.Cu") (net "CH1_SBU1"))
 (segment (start 62.0483 35.0034) (end 62.45 34.6017) (width 0.2) (layer "F.Cu") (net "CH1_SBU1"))
 (segment (start 46.45 34) (end 47.0517 34) (width 0.2) (layer "F.Cu") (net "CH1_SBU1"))
 (segment (start 36.889 41.329) (end 36.9583 41.3983) (width 0.2) (layer "F.Cu") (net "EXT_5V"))
 (segment (start 61.55 50) (end 60.9483 50) (width 0.2) (layer "F.Cu") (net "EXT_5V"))
 (segment (start 44.3983 42) (end 43.7966 41.3983) (width 0.2) (layer "F.Cu") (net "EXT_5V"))
 (segment (start 37.55 42) (end 37.2492 42) (width 0.2) (layer "F.Cu") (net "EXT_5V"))
 (segment (start 45.1 42) (end 44.3983 42) (width 0.2) (layer "F.Cu") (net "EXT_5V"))
 (segment (start 44.9483 49.6991) (end 44.9483 50) (width 0.2) (layer "F.Cu") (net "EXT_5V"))
 (segment (start 45.55 50.6017) (end 60.3466 50.6017) (width 0.2) (layer "F.Cu") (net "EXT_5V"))
 (segment (start 45.55 50) (end 45.55 50.6017) (width 0.2) (layer "F.Cu") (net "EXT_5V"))
 (segment (start 43.7966 41.3983) (end 36.9583 41.3983) (width 0.2) (layer "F.Cu") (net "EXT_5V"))
 (segment (start 36.9583 41.3983) (end 36.9483 41.4083) (width 0.2) (layer "F.Cu") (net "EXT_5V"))
 (segment (start 45.55 50) (end 44.9483 50) (width 0.2) (layer "F.Cu") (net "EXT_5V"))
 (segment (start 60.3466 50.6017) (end 60.9483 50) (width 0.2) (layer "F.Cu") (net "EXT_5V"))
 (segment (start 37.2492 42) (end 44.9483 49.6991) (width 0.2) (layer "F.Cu") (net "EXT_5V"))
 (segment (start 36.9483 41.4083) (end 36.9483 42) (width 0.2) (layer "F.Cu") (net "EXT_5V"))
 (segment (start 37.2492 42) (end 36.9483 42) (width 0.2) (layer "F.Cu") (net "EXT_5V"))
 (via (at 36.889 41.329) (size 0.6) (drill 0.3) (layers "F.Cu" "B.Cu") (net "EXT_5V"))
 (segment (start 30.81 35.27) (end 30.83 35.27) (width 0.2) (layer "B.Cu") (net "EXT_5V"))
 (segment (start 30.81 35.27) (end 29.54 34) (width 0.2) (layer "B.Cu") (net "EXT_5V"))
 (segment (start 24.46 34) (end 23.19 32.73) (width 0.2) (layer "B.Cu") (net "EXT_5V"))
 (segment (start 29.54 34) (end 24.46 34) (width 0.2) (layer "B.Cu") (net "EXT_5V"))
 (segment (start 30.83 35.27) (end 36.889 41.329) (width 0.2) (layer "B.Cu") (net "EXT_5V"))
 (segment (start 59.05 33.1227) (end 60.071 33.1227) (width 0.2) (layer "F.Cu") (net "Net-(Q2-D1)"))
 (segment (start 61.05 23.7982) (end 60.3444 23.7982) (width 0.2) (layer "F.Cu") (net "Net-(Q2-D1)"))
 (segment (start 61.05 24.6999) (end 61.05 23.7982) (width 0.2) (layer "F.Cu") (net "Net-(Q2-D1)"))
 (segment (start 61.55 34) (end 60.9483 34) (width 0.2) (layer "F.Cu") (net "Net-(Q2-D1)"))
 (segment (start 60.071 33.1227) (end 60.9483 34) (width 0.2) (layer "F.Cu") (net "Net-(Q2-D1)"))
 (via (at 59.05 33.1227) (size 0.6) (drill 0.3) (layers "F.Cu" "B.Cu") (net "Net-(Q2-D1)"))
 (via (at 60.3444 23.7982) (size 0.6) (drill 0.3) (layers "F.Cu" "B.Cu") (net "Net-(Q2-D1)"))
 (segment (start 59.05 25.0926) (end 60.3444 23.7982) (width 0.2) (layer "B.Cu") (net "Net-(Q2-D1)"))
 (segment (start 59.05 33.1227) (end 59.05 25.0926) (width 0.2) (layer "B.Cu") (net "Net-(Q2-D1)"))
 (segment (start 54 27.05) (end 50.8282 27.05) (width 0.2) (layer "F.Cu") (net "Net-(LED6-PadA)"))
 (segment (start 46.45 50) (end 49.8886 50) (width 0.2) (layer "F.Cu") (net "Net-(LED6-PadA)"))
 (via (at 50.8282 27.05) (size 0.6) (drill 0.3) (layers "F.Cu" "B.Cu") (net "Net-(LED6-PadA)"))
 (via (at 49.8886 50) (size 0.6) (drill 0.3) (layers "F.Cu" "B.Cu") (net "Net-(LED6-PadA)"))
 (segment (start 50.8282 27.05) (end 50.8282 49.0604) (width 0.2) (layer "B.Cu") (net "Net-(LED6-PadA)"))
 (segment (start 50.8282 49.0604) (end 49.8886 50) (width 0.2) (layer "B.Cu") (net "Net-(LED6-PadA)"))
 (segment (start 57.5908 27.3001) (end 56.4265 26.1358) (width 0.2) (layer "F.Cu") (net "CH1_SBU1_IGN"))
 (segment (start 54.45 50) (end 54.45 49.3983) (width 0.2) (layer "F.Cu") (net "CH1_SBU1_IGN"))
 (segment (start 39.4634 26.2367) (end 40.2398 27.0131) (width 0.2) (layer "F.Cu") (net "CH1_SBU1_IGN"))
 (segment (start 40.2398 27.0131) (end 46.6511 27.0131) (width 0.2) (layer "F.Cu") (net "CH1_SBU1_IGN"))
 (segment (start 45.55 26) (end 45.55 25.3983) (width 0.2) (layer "F.Cu") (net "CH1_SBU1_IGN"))
 (segment (start 47.0548 26.6094) (end 47.0548 26.1358) (width 0.2) (layer "F.Cu") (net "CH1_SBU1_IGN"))
 (segment (start 24.46 32.2004) (end 30.4237 26.2367) (width 0.2) (layer "F.Cu") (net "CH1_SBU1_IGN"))
 (segment (start 47.0548 25.5712) (end 47.0548 26.1358) (width 0.2) (layer "F.Cu") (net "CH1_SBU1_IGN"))
 (segment (start 25.73 35.27) (end 24.46 34) (width 0.2) (layer "F.Cu") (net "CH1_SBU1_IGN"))
 (segment (start 46.6511 27.0131) (end 47.0548 26.6094) (width 0.2) (layer "F.Cu") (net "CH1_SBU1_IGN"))
 (segment (start 46.8819 25.3983) (end 47.0548 25.5712) (width 0.2) (layer "F.Cu") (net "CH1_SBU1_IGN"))
 (segment (start 61.05 27.3001) (end 57.5908 27.3001) (width 0.2) (layer "F.Cu") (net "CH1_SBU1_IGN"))
 (segment (start 56.4265 26.1358) (end 47.0548 26.1358) (width 0.2) (layer "F.Cu") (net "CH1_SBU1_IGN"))
 (segment (start 45.55 25.3983) (end 46.8819 25.3983) (width 0.2) (layer "F.Cu") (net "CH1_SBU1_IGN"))
 (segment (start 24.46 34) (end 24.46 32.2004) (width 0.2) (layer "F.Cu") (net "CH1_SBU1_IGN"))
 (segment (start 30.4237 26.2367) (end 39.4634 26.2367) (width 0.2) (layer "F.Cu") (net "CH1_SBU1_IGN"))
 (segment (start 54.7895 49.1757) (end 54.5669 49.3983) (width 0.2) (layer "F.Cu") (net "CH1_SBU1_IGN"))
 (segment (start 54.5669 49.3983) (end 54.45 49.3983) (width 0.2) (layer "F.Cu") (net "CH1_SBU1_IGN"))
 (via (at 54.7895 49.1757) (size 0.6) (drill 0.3) (layers "F.Cu" "B.Cu") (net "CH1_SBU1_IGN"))
 (via (at 57.5908 27.3001) (size 0.6) (drill 0.3) (layers "F.Cu" "B.Cu") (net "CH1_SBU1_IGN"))
 (segment (start 54.7895 30.1014) (end 57.5908 27.3001) (width 0.2) (layer "B.Cu") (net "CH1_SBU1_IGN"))
 (segment (start 54.7895 49.1757) (end 54.7895 30.1014) (width 0.2) (layer "B.Cu") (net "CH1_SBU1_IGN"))
 (segment (start 28.27 32.73) (end 29.5409 31.4591) (width 0.2) (layer "F.Cu") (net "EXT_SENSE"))
 (segment (start 45.55 34) (end 44.9483 34) (width 0.2) (layer "F.Cu") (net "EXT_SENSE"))
 (segment (start 29.5409 31.4591) (end 42.4074 31.4591) (width 0.2) (layer "F.Cu") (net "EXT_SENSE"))
 (segment (start 42.4074 31.4591) (end 44.9483 34) (width 0.2) (layer "F.Cu") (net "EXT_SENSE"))
 (segment (start 37.05 27) (end 37.7517 27) (width 0.2) (layer "F.Cu") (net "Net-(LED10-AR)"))
 (segment (start 50.7635 47.8152) (end 52.9483 50) (width 0.2) (layer "F.Cu") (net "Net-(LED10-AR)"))
 (segment (start 44.55 47.8152) (end 50.7635 47.8152) (width 0.2) (layer "F.Cu") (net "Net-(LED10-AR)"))
 (segment (start 37.7517 27) (end 37.9567 27) (width 0.2) (layer "F.Cu") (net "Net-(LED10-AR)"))
 (segment (start 53.55 50) (end 52.9483 50) (width 0.2) (layer "F.Cu") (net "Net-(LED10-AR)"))
 (via (at 44.55 47.8152) (size 0.6) (drill 0.3) (layers "F.Cu" "B.Cu") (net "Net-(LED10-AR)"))
 (via (at 37.9567 27) (size 0.6) (drill 0.3) (layers "F.Cu" "B.Cu") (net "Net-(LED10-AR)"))
 (segment (start 44.55 47.8152) (end 44.55 33.5933) (width 0.2) (layer "B.Cu") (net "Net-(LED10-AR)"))
 (segment (start 44.55 33.5933) (end 37.9567 27) (width 0.2) (layer "B.Cu") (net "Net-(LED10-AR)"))
 (segment (start 52.9483 34) (end 46.65 27.7017) (width 0.2) (layer "F.Cu") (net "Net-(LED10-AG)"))
 (segment (start 38.95 27) (end 39.6517 27) (width 0.2) (layer "F.Cu") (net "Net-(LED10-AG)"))
 (segment (start 53.55 34) (end 52.9483 34) (width 0.2) (layer "F.Cu") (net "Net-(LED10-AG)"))
 (segment (start 46.65 27.7017) (end 40.3534 27.7017) (width 0.2) (layer "F.Cu") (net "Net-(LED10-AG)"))
 (segment (start 40.3534 27.7017) (end 39.6517 27) (width 0.2) (layer "F.Cu") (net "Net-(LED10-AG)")))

